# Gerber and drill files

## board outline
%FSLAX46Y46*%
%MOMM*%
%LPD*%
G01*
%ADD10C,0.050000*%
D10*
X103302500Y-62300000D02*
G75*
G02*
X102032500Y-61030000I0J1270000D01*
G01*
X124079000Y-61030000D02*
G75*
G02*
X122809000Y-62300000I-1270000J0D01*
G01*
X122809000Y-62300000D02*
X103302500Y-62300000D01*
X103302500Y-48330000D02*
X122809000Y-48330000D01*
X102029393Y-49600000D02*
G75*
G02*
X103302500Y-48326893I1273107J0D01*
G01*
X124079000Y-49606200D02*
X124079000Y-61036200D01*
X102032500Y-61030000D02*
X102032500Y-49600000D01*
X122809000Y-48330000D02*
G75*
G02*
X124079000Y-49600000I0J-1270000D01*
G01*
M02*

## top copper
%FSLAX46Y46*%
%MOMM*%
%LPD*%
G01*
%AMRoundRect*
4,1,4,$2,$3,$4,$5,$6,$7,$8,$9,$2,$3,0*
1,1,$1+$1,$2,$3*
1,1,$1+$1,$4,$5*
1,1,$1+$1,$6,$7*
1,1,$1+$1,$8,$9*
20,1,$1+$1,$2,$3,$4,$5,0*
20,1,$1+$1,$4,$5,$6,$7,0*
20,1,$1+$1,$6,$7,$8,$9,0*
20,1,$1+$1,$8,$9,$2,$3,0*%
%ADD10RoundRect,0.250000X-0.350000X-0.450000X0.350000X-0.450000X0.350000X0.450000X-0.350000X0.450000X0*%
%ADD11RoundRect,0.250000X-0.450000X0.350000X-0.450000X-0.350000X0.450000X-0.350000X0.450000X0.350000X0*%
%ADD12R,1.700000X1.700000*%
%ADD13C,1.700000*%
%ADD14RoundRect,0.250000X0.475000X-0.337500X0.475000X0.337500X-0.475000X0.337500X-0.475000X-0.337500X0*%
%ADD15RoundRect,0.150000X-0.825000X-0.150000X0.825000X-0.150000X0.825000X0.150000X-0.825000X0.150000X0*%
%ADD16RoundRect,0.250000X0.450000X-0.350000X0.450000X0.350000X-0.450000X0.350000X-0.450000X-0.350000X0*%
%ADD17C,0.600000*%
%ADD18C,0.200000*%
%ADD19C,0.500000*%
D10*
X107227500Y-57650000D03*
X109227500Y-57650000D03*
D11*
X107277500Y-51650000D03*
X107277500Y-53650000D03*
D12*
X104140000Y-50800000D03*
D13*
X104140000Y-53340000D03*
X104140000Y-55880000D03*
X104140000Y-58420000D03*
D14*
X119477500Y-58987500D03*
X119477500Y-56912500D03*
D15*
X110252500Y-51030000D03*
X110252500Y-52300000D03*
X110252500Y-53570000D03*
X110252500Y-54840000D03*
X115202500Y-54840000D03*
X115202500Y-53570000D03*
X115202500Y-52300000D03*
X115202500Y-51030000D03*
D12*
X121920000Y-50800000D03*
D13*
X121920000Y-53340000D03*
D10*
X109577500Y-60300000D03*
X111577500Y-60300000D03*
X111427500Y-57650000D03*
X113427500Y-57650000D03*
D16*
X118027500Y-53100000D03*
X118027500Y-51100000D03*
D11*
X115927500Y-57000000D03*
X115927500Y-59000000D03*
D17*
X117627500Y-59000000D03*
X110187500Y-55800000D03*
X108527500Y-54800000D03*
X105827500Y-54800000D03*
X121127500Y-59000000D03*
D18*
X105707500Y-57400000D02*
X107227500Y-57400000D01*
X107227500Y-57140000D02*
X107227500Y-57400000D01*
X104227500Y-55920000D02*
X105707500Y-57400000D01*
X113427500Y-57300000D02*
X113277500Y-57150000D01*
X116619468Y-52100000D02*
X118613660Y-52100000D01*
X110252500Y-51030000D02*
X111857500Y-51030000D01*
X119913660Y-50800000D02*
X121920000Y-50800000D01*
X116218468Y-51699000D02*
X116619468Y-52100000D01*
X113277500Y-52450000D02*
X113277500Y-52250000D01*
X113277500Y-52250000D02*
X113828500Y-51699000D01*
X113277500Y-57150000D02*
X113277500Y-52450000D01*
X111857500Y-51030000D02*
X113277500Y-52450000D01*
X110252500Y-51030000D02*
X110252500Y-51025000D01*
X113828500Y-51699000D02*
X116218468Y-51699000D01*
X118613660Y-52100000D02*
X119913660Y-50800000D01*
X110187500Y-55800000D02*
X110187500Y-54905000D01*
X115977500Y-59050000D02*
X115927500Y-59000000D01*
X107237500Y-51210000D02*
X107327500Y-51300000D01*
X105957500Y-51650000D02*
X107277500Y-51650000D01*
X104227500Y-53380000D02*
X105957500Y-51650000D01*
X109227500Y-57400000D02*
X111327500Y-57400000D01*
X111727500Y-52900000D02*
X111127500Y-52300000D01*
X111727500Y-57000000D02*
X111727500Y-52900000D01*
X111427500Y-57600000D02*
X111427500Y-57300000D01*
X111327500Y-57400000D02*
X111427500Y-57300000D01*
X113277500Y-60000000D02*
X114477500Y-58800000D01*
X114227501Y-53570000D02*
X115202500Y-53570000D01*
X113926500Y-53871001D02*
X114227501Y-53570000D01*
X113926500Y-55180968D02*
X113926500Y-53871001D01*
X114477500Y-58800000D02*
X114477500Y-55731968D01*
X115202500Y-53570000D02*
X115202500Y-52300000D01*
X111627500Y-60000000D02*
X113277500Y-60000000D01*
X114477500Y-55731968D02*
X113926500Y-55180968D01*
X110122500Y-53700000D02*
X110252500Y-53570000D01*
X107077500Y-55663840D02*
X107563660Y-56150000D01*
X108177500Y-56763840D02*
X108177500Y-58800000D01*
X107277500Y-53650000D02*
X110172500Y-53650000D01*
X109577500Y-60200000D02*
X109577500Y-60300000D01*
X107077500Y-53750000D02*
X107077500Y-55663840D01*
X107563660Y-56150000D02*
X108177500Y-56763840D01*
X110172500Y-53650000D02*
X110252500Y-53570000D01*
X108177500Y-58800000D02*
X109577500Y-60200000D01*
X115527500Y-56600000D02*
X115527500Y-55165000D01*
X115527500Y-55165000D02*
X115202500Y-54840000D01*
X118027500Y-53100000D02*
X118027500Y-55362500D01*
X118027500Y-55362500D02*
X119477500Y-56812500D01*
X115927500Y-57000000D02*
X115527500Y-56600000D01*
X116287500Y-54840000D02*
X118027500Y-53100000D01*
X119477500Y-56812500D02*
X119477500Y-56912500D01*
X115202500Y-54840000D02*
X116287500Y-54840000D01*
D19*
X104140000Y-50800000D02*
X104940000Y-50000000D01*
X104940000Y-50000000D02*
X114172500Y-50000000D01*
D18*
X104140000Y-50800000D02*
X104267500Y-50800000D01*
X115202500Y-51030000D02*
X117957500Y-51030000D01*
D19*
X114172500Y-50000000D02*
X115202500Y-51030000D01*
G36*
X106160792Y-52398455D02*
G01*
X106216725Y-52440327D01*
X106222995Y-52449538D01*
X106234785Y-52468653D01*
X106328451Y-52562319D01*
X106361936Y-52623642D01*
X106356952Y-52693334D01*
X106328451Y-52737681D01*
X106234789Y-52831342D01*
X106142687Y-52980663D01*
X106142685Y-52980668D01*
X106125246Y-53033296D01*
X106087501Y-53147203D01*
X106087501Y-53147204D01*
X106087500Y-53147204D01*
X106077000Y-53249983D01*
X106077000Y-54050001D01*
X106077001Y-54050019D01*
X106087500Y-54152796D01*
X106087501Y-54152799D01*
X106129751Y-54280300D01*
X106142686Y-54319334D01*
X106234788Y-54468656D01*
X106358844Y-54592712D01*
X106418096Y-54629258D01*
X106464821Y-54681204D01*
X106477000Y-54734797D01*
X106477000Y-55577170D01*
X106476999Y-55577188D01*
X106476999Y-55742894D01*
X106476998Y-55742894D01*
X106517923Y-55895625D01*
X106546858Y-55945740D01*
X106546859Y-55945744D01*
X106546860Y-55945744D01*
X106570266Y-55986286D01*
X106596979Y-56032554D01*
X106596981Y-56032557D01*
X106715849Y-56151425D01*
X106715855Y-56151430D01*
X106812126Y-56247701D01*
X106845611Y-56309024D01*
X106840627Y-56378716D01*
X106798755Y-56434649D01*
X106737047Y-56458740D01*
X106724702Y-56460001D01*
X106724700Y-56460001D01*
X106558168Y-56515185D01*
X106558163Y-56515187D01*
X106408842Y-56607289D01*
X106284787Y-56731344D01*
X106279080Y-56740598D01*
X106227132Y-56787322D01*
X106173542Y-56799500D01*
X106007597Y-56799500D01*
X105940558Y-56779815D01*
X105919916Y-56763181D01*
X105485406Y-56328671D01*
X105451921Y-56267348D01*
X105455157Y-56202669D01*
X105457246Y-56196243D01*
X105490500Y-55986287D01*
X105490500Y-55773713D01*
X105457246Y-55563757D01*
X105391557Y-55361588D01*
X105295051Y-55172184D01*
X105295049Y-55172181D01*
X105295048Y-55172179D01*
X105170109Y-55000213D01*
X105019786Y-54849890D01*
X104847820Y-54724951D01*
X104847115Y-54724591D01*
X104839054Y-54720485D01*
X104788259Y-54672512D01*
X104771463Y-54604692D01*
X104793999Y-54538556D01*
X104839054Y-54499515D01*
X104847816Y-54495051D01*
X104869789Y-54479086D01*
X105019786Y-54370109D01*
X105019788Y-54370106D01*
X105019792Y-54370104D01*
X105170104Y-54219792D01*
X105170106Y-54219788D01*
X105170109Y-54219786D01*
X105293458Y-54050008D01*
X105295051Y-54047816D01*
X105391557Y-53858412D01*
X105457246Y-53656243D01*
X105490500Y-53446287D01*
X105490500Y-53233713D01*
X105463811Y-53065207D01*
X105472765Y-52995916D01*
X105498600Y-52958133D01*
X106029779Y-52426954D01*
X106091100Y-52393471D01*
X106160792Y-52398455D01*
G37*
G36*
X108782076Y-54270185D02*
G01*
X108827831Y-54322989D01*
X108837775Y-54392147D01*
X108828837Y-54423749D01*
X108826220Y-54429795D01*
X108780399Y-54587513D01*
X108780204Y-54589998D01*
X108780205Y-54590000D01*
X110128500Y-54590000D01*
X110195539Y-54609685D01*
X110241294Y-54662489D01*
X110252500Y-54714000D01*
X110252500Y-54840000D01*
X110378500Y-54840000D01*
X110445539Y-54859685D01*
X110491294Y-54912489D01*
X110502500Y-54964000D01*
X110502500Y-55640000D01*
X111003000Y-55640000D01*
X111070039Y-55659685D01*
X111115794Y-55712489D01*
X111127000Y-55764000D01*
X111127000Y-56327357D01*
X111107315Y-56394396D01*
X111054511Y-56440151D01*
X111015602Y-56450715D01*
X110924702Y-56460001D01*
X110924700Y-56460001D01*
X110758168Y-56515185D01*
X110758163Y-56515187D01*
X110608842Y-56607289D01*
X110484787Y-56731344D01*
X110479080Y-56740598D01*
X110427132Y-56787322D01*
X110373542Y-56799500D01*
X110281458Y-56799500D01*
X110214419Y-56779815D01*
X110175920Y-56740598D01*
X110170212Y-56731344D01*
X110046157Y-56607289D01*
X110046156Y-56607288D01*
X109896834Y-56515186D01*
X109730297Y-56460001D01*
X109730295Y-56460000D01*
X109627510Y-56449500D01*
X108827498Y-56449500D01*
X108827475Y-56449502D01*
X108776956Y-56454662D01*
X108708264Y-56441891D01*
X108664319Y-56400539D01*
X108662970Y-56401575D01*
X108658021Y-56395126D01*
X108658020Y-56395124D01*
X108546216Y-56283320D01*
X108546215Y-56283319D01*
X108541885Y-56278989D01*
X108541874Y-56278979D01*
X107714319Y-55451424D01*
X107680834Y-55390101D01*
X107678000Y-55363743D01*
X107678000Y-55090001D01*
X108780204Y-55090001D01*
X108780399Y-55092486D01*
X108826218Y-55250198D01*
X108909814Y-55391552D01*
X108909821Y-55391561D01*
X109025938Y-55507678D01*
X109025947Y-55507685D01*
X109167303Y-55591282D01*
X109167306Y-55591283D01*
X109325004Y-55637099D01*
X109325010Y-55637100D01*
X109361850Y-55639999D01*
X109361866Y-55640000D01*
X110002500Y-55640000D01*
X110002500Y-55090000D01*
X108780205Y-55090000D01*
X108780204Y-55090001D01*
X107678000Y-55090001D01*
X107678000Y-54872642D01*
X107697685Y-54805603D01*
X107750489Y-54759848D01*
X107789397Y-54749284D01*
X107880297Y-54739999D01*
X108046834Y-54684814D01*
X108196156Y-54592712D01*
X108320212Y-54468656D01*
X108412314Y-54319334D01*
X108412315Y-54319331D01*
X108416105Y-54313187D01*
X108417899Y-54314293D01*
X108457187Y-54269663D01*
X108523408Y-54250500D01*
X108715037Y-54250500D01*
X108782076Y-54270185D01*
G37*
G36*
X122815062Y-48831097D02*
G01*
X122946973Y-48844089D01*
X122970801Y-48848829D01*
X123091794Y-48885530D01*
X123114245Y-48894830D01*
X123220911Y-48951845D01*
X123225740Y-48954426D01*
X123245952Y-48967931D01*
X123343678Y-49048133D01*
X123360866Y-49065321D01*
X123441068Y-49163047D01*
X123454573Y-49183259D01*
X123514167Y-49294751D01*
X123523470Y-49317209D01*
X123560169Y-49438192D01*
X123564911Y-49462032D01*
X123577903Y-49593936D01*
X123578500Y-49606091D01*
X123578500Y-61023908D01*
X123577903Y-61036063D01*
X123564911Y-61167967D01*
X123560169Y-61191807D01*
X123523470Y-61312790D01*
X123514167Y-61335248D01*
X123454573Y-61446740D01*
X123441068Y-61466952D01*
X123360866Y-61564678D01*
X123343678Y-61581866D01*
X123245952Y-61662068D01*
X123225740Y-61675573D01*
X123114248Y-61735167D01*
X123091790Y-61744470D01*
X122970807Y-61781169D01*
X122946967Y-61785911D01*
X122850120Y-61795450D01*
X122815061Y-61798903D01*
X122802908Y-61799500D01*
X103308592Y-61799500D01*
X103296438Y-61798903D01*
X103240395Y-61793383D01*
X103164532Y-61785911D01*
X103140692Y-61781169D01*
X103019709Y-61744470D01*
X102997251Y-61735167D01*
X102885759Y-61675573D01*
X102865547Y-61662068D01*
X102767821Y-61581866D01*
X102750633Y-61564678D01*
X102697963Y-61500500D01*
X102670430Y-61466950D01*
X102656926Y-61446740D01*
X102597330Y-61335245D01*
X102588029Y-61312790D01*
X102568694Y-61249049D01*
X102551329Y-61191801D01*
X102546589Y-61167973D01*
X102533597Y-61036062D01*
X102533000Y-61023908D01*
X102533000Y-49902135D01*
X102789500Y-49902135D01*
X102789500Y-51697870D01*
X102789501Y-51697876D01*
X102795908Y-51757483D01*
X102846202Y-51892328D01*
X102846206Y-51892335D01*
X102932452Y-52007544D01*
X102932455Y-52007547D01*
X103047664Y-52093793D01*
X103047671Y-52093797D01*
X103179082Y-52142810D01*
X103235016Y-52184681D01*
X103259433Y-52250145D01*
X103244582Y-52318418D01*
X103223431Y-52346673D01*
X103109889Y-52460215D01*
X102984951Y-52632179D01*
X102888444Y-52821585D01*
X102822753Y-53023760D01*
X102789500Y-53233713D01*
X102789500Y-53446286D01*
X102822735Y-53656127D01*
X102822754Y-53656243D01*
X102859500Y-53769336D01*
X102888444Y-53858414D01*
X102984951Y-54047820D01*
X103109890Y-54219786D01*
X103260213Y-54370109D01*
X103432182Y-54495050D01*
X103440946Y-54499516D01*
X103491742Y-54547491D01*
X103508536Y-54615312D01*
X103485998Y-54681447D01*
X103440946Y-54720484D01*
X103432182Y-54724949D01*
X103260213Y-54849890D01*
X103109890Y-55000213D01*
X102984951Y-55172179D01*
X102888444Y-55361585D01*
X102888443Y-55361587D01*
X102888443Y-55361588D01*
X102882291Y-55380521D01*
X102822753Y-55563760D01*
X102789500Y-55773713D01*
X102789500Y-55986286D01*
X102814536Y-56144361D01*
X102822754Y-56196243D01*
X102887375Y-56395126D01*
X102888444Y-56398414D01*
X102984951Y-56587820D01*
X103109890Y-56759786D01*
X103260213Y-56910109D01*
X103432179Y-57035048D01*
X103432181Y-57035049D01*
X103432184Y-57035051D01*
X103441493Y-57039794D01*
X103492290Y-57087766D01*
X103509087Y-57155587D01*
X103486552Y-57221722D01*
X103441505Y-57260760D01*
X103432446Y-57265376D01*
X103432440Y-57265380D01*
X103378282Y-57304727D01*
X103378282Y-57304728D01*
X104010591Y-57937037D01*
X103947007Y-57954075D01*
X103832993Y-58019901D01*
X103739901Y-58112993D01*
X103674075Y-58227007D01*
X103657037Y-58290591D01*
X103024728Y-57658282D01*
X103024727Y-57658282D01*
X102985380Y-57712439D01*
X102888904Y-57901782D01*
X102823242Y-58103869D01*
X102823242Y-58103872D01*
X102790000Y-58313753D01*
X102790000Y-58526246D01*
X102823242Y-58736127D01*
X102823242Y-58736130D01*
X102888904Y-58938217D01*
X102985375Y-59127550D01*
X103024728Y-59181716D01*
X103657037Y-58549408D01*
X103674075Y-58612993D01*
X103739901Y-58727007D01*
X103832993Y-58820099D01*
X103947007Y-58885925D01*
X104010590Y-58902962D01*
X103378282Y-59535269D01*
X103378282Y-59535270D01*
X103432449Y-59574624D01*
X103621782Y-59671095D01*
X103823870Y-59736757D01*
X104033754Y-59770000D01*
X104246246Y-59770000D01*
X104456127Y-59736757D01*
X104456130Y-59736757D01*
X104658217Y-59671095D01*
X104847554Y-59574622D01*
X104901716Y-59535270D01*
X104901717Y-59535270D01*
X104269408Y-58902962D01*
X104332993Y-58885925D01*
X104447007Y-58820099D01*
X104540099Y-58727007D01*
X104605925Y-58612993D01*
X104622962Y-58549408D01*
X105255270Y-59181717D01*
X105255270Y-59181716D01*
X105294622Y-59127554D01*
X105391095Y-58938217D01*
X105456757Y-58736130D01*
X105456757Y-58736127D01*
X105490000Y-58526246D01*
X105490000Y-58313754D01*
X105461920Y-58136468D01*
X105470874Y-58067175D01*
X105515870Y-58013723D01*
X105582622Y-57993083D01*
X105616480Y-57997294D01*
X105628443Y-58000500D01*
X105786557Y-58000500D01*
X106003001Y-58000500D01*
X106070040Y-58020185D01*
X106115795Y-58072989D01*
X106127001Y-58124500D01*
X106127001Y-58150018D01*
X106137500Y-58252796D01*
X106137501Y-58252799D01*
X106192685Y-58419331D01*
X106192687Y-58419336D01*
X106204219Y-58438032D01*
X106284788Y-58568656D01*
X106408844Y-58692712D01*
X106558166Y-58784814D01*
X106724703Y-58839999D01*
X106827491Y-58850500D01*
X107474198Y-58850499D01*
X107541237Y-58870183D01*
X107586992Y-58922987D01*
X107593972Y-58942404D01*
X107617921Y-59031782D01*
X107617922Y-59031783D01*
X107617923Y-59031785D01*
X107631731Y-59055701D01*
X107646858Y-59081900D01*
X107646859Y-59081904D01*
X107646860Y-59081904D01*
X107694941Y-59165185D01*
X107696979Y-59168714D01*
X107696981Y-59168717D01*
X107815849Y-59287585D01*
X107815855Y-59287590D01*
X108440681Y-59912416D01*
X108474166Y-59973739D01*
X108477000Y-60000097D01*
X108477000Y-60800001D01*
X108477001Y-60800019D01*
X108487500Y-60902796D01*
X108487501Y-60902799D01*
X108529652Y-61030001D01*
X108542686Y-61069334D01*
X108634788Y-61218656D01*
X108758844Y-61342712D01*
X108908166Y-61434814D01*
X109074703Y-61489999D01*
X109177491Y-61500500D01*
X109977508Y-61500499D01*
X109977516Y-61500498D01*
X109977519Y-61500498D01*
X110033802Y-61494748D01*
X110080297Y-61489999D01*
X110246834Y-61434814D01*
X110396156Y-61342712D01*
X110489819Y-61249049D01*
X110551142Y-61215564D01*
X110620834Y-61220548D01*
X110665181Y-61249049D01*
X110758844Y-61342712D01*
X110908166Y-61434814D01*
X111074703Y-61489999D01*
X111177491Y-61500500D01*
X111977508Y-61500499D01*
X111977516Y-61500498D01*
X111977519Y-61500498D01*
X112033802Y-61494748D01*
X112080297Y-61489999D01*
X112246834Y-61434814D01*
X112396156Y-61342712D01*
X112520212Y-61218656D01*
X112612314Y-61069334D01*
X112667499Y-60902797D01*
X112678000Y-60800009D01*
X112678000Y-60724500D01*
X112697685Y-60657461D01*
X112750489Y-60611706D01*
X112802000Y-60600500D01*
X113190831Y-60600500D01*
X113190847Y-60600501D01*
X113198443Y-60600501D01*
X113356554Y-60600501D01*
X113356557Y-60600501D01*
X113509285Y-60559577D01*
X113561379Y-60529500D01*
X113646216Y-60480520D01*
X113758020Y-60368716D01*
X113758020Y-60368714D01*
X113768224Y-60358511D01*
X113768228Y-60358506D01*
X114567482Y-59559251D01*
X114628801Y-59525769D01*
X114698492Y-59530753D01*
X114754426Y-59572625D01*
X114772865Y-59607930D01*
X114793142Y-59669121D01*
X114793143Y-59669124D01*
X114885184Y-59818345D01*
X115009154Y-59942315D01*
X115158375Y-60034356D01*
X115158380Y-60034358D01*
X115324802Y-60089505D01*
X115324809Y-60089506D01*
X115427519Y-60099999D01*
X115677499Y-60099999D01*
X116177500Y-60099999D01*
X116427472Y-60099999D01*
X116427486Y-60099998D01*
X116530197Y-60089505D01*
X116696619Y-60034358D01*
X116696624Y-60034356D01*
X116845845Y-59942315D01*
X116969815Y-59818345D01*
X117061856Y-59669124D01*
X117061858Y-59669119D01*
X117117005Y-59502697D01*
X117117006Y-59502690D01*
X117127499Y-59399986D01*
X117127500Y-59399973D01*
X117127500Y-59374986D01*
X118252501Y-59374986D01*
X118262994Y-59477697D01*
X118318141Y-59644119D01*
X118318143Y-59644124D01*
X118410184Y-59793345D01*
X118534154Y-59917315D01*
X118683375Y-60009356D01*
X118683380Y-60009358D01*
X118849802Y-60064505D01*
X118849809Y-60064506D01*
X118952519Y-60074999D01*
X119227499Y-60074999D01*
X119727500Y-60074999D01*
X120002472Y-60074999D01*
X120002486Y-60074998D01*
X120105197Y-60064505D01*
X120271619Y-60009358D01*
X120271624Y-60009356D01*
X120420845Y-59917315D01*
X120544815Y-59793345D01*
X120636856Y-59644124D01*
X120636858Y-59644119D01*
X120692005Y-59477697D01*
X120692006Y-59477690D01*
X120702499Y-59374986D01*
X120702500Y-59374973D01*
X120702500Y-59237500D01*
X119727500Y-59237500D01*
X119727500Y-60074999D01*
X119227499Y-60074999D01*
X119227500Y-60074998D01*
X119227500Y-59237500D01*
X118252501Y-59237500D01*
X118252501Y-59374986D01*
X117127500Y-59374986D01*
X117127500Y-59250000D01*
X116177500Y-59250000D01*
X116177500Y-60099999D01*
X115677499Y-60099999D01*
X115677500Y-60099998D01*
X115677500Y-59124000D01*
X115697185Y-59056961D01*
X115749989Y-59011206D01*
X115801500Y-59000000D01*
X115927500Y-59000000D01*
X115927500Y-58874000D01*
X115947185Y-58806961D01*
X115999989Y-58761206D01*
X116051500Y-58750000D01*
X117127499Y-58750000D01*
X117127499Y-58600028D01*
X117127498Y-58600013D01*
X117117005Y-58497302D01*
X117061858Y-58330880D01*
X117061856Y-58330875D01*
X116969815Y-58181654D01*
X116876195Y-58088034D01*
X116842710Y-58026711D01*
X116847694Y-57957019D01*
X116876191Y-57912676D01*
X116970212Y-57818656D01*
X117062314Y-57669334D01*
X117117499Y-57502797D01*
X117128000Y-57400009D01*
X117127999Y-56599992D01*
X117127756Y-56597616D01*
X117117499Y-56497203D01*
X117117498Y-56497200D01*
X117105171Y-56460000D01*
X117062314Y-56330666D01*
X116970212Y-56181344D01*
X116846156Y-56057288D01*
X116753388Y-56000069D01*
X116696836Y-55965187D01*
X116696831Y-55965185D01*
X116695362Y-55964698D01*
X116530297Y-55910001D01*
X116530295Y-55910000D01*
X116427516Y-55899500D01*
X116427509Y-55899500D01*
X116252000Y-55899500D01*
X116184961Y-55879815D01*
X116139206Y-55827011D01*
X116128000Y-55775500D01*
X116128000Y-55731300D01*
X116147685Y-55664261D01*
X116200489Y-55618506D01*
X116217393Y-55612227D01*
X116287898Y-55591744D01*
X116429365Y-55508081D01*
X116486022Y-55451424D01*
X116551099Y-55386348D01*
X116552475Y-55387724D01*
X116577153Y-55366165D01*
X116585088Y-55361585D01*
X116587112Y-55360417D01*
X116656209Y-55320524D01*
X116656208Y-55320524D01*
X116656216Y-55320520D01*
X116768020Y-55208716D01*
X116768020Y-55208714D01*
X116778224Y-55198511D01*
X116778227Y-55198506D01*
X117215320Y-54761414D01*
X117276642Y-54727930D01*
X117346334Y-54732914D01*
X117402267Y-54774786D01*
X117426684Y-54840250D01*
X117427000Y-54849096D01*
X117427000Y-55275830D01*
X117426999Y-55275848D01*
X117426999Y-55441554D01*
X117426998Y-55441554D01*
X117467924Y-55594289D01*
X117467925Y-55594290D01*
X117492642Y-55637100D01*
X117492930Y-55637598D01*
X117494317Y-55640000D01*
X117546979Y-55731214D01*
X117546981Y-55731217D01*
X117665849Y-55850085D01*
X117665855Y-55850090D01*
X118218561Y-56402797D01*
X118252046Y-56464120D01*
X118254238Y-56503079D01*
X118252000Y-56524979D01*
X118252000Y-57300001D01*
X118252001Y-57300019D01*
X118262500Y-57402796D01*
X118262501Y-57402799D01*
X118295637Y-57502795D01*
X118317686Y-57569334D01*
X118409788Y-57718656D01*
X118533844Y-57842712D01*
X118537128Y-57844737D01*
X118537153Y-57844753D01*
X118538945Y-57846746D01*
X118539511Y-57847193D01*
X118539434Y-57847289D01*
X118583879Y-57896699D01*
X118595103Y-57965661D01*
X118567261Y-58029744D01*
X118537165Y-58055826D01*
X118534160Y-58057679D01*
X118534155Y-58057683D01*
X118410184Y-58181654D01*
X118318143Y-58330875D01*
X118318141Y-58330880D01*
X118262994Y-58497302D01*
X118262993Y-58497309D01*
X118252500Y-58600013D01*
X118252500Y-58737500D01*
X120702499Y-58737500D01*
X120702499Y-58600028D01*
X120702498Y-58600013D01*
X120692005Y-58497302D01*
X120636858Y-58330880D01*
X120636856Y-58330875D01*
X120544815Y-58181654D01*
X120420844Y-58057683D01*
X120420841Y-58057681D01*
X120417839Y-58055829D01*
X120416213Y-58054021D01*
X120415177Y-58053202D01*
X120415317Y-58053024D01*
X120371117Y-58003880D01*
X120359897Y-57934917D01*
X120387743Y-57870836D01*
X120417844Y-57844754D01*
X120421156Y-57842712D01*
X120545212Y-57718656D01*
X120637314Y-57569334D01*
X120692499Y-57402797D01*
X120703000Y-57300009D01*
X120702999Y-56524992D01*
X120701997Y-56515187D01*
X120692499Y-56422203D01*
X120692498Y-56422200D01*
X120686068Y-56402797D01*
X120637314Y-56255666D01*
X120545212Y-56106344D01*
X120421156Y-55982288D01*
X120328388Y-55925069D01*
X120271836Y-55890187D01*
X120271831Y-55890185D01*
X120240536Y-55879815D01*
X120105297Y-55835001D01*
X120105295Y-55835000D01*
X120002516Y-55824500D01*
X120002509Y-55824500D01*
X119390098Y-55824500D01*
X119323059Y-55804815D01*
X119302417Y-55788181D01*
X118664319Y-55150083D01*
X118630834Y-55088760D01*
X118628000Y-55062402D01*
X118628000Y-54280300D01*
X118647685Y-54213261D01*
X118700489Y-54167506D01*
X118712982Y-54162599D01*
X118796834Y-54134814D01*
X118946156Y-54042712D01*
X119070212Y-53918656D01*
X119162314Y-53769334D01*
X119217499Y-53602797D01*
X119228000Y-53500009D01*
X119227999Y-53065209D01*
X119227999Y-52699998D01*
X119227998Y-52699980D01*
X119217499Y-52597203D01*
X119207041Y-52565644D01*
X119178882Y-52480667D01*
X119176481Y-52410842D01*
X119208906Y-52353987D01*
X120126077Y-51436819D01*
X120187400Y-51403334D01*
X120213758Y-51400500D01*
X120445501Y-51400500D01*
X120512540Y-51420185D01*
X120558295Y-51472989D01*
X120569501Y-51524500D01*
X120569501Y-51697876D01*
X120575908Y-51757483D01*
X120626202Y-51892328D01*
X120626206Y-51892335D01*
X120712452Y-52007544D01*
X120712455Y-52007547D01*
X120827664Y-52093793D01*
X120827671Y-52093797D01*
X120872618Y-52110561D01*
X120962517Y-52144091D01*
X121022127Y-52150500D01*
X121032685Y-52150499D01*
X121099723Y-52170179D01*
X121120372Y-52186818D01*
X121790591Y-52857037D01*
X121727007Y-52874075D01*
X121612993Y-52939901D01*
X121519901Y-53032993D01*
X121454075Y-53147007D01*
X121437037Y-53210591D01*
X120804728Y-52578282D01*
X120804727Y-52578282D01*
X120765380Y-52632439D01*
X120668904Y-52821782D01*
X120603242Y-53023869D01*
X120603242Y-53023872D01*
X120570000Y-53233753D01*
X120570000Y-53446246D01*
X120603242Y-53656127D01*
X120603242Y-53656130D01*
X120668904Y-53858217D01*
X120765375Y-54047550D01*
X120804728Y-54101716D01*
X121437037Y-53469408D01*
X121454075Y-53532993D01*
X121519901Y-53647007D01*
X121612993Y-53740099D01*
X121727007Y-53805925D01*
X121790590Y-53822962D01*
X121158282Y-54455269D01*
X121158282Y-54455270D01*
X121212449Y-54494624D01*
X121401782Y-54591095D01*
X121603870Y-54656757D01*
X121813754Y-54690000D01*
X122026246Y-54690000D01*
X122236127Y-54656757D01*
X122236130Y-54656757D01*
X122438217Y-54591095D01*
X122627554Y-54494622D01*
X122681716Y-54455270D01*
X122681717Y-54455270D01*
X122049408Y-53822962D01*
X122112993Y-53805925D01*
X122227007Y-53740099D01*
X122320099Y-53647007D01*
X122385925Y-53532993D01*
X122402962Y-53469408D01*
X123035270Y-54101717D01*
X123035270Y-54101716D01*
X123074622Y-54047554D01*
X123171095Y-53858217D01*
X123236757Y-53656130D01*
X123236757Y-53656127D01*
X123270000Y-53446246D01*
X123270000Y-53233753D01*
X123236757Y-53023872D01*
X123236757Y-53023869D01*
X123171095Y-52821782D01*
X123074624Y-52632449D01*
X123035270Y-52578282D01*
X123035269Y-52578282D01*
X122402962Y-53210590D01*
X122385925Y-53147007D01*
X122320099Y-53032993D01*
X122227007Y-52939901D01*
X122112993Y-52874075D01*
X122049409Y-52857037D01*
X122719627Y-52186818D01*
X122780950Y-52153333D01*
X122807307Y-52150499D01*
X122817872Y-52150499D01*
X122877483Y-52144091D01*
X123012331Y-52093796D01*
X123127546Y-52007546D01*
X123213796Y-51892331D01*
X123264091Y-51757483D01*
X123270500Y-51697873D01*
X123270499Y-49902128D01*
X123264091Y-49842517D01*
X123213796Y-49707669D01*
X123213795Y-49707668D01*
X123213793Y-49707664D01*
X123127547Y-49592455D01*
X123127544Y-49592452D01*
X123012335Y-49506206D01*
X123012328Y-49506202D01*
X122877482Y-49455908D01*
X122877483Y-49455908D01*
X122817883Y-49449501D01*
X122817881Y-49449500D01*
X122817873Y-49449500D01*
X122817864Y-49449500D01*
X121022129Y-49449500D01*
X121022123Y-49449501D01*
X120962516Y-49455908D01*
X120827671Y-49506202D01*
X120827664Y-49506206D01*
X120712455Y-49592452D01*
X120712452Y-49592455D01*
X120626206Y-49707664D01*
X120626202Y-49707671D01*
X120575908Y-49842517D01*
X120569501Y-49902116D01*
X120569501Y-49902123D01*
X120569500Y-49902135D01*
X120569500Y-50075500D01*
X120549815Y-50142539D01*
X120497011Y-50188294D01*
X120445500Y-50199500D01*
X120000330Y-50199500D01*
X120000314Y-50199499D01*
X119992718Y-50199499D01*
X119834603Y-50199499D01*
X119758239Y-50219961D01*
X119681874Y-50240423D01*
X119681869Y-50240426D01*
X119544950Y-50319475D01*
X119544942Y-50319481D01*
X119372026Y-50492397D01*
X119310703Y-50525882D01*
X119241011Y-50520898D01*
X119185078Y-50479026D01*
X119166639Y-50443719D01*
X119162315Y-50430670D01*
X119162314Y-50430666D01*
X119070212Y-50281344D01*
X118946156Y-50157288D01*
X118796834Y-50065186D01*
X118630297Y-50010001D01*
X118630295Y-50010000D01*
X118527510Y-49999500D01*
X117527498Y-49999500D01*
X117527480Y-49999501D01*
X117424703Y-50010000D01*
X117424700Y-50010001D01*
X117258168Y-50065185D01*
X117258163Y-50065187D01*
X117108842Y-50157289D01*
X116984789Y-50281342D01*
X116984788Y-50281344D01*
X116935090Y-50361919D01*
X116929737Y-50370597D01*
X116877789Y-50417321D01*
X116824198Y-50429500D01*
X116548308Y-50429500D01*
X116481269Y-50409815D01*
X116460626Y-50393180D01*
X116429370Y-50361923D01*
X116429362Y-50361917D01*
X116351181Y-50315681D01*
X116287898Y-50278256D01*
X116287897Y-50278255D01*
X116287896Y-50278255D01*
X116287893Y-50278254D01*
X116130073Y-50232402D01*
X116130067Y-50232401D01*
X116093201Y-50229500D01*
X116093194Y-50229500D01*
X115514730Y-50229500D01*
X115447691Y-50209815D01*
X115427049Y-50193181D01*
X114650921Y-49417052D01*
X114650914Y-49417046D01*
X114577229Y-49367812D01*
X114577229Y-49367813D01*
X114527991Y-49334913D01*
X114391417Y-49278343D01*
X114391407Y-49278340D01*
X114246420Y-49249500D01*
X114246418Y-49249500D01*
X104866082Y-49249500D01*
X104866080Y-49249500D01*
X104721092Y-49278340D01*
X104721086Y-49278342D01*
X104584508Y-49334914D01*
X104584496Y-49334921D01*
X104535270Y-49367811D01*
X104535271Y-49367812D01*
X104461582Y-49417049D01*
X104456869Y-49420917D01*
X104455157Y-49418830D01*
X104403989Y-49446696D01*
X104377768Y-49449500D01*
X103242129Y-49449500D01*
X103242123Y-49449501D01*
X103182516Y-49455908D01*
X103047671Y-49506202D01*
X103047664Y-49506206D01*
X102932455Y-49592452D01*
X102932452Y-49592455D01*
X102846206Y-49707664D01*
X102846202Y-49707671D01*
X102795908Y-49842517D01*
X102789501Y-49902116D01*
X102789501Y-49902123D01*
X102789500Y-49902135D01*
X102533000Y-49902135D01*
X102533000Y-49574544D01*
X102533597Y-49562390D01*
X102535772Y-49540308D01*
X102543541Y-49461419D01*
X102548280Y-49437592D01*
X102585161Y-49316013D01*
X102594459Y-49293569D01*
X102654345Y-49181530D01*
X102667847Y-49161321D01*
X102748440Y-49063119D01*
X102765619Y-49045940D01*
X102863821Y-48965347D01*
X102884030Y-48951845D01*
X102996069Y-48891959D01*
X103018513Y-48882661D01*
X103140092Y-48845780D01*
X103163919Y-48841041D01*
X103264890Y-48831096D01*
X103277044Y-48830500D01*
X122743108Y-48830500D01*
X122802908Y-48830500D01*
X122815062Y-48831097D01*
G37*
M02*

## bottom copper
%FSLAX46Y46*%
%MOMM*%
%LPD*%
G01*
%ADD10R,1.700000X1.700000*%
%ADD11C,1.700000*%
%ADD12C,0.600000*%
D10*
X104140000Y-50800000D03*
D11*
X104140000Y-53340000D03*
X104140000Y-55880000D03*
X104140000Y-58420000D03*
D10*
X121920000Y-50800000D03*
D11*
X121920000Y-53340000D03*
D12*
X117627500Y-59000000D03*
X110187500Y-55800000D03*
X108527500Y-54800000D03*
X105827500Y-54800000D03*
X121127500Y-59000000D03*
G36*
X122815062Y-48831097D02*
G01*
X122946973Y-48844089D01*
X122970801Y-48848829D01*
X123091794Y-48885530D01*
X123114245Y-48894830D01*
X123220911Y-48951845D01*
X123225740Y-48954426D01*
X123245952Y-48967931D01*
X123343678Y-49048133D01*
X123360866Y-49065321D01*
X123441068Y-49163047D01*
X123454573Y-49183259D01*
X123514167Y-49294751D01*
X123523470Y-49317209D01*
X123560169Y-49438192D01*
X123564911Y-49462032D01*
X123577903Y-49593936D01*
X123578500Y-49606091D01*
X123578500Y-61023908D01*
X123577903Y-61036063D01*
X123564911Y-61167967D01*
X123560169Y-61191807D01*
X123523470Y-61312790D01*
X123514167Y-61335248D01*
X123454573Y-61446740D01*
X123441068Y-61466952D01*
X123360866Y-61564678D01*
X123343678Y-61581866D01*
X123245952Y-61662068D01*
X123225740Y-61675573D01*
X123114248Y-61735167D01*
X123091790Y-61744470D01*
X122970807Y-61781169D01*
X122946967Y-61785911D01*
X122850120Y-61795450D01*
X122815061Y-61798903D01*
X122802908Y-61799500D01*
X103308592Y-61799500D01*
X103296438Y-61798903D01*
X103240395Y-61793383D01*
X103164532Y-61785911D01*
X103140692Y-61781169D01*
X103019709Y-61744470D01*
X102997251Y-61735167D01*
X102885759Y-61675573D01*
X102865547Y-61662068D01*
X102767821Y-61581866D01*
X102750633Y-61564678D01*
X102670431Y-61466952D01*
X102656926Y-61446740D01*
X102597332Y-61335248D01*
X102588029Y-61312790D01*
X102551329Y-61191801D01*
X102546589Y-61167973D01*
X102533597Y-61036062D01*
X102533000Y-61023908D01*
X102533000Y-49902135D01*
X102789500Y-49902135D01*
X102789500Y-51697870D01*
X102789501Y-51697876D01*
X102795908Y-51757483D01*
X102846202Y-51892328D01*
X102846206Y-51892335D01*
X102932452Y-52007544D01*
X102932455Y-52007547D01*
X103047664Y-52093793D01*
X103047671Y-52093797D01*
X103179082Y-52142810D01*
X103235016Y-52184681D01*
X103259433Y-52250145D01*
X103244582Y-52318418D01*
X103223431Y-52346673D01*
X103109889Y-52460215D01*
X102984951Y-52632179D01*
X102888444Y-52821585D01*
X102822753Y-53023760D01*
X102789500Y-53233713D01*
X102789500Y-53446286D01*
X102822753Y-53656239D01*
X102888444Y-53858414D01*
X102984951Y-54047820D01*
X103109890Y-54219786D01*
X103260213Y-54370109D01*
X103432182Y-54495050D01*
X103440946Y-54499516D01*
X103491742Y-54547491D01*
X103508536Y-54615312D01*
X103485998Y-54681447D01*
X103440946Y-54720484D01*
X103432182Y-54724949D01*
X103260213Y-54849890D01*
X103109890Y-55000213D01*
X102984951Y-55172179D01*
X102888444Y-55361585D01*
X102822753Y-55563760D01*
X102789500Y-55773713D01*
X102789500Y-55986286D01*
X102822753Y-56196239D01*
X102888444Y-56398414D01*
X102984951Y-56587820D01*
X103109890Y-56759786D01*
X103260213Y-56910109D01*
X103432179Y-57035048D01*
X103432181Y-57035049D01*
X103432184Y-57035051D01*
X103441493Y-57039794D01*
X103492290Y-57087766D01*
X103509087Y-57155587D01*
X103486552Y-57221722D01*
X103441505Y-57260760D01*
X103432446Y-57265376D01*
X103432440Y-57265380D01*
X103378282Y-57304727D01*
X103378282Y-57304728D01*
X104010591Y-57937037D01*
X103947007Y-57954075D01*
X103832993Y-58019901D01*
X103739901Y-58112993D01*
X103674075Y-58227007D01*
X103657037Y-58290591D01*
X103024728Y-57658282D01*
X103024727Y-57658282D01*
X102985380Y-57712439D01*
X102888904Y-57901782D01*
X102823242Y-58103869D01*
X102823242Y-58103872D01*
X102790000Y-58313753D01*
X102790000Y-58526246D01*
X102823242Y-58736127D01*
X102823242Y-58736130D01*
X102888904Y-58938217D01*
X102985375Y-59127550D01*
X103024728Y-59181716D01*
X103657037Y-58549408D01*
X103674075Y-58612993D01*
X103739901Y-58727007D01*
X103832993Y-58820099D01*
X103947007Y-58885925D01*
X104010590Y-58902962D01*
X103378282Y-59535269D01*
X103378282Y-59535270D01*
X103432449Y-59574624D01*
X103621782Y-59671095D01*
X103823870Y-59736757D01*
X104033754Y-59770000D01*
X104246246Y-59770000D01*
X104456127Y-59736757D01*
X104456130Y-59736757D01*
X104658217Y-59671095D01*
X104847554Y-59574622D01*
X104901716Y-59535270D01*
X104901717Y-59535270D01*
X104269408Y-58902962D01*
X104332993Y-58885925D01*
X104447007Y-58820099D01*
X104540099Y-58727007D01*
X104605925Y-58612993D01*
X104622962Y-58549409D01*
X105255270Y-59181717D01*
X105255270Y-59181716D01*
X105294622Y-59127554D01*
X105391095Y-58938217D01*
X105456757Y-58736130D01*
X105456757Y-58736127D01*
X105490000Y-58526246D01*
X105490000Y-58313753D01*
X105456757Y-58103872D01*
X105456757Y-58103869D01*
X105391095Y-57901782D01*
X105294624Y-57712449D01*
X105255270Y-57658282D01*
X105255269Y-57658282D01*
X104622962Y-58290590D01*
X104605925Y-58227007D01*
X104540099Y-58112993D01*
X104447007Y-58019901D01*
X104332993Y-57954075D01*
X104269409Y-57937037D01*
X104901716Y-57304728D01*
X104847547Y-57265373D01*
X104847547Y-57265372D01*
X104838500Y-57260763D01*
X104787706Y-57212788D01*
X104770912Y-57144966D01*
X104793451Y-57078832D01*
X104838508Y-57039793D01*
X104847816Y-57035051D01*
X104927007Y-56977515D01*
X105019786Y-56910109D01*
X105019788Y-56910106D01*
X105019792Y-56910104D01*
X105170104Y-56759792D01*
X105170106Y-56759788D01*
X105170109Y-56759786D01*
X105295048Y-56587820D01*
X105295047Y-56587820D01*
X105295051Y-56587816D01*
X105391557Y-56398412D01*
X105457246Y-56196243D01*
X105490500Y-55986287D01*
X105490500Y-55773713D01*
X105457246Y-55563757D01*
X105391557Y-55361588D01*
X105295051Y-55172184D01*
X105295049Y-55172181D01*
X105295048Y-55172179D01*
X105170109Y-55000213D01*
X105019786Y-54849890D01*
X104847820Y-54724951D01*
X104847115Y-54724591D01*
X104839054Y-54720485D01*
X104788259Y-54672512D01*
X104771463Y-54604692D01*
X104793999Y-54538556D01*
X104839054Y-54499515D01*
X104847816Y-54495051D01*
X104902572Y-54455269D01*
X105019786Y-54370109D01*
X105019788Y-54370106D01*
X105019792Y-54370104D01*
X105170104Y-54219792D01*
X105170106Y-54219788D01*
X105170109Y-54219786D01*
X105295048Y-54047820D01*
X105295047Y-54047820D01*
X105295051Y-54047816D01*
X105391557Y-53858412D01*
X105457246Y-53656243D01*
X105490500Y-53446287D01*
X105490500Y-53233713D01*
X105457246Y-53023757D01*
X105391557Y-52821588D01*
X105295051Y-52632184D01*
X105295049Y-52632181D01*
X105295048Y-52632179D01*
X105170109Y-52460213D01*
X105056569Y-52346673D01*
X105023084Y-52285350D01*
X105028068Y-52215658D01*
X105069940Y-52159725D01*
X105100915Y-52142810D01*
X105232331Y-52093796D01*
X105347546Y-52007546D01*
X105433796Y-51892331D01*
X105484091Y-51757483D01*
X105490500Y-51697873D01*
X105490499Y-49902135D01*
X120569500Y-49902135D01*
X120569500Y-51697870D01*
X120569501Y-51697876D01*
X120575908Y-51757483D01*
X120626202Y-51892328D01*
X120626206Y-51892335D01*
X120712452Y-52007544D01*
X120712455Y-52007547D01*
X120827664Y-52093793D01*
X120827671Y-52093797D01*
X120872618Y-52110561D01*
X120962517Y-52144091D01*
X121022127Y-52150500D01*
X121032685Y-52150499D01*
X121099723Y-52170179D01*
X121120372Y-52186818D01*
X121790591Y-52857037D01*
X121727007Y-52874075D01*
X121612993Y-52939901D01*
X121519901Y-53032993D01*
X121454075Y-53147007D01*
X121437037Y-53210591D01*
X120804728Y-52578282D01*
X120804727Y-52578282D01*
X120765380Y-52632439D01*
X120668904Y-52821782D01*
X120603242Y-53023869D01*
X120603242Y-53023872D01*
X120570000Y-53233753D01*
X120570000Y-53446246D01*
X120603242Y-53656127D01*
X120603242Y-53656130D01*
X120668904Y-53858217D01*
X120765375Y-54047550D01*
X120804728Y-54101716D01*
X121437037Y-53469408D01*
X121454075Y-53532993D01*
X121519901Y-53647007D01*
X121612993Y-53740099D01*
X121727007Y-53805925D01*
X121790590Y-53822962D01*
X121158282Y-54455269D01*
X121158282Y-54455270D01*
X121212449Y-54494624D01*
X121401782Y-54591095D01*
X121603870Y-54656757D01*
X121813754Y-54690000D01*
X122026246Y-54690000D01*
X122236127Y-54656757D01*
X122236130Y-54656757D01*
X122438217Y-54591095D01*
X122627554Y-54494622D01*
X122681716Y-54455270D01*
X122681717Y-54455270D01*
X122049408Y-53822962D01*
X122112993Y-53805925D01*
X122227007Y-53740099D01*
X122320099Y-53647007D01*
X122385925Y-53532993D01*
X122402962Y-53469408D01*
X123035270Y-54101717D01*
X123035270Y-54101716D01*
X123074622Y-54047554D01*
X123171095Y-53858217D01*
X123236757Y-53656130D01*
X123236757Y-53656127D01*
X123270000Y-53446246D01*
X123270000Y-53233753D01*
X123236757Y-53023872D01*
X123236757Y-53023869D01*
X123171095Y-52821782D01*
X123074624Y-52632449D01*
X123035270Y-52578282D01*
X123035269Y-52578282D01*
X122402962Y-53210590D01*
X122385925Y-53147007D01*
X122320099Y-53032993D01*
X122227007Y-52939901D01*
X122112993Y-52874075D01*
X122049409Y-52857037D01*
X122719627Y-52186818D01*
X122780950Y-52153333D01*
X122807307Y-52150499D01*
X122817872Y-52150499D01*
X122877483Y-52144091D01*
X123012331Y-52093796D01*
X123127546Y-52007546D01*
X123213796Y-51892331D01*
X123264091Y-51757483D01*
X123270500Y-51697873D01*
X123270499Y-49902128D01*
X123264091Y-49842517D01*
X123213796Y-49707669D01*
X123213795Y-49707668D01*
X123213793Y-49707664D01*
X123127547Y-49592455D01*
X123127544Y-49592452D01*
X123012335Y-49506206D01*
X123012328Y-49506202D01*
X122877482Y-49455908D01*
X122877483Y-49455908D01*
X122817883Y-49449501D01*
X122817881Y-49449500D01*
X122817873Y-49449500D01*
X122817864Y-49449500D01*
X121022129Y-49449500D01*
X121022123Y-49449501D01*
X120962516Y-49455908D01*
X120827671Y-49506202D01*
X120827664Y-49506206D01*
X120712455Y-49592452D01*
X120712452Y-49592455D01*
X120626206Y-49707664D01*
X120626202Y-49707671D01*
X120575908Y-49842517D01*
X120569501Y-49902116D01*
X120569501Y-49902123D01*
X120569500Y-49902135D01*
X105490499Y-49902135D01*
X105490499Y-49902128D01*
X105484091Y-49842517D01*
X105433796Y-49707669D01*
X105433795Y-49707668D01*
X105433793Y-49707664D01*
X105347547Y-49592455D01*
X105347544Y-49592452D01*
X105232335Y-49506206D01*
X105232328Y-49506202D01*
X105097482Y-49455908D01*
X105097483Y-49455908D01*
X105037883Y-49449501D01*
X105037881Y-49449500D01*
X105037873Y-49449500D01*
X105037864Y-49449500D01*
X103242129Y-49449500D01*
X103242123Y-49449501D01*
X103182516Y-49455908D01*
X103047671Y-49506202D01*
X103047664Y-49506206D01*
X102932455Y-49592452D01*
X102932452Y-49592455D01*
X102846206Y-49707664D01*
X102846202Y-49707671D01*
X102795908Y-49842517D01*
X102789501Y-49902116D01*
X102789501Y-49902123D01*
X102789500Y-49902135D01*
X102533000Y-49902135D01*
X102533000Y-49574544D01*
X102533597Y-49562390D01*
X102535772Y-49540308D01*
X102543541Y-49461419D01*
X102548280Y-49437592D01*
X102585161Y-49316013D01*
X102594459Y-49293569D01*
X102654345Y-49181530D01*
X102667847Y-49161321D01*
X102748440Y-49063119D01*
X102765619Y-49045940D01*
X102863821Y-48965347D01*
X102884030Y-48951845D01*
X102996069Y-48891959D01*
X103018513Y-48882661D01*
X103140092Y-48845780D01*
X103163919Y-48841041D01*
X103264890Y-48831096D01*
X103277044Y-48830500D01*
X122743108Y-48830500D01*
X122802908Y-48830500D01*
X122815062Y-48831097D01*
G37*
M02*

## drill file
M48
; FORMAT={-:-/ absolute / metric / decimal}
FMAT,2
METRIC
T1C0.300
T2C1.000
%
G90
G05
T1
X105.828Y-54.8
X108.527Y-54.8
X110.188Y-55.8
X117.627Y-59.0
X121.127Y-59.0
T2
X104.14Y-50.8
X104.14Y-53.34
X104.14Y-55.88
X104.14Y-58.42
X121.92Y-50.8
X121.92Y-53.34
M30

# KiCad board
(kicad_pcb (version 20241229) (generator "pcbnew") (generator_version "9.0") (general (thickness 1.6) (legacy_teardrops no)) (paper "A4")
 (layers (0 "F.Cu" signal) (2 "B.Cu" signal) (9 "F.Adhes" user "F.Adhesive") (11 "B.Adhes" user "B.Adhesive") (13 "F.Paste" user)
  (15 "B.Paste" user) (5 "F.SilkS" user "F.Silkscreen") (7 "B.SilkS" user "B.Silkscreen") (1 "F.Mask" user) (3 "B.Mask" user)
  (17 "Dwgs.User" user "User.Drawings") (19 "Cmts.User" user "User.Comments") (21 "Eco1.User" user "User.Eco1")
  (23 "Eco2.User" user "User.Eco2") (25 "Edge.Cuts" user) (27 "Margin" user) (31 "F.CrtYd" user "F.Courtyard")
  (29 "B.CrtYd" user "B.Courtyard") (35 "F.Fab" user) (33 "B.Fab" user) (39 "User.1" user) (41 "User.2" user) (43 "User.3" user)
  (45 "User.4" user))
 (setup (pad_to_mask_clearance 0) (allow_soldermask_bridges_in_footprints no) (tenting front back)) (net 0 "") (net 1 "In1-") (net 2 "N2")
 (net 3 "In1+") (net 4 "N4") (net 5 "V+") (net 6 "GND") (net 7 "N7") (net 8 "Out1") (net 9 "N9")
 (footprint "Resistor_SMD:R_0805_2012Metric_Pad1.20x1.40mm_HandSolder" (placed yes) (layer "F.Cu") (at 108.2275 57.65)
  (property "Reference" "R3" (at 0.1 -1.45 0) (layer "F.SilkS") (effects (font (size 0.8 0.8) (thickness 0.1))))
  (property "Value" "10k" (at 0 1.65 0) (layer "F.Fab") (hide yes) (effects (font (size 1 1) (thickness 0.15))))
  (pad "1" smd roundrect (at -1 0) (size 1.2 1.4) (layers "F.Cu" "F.Mask" "F.Paste") (roundrect_rratio 0.208333) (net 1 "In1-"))
  (pad "2" smd roundrect (at 1 0) (size 1.2 1.4) (layers "F.Cu" "F.Mask" "F.Paste") (roundrect_rratio 0.208333) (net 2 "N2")))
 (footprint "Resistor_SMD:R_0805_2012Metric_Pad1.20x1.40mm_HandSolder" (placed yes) (layer "F.Cu") (at 107.2775 52.65 -90)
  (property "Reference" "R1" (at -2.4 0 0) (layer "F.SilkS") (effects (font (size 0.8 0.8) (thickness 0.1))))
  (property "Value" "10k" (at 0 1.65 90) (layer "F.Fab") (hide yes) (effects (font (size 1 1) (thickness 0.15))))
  (pad "1" smd roundrect (at -1 0 270) (size 1.2 1.4) (layers "F.Cu" "F.Mask" "F.Paste") (roundrect_rratio 0.208333) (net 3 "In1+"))
  (pad "2" smd roundrect (at 1 0 270) (size 1.2 1.4) (layers "F.Cu" "F.Mask" "F.Paste") (roundrect_rratio 0.208333) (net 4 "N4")))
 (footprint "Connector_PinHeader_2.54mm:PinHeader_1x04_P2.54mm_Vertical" (layer "F.Cu") (at 104.14 50.8)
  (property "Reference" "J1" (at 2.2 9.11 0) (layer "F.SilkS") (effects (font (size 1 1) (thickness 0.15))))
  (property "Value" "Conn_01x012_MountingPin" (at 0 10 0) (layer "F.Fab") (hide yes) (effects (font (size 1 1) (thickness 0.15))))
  (pad "1" thru_hole rect (at 0 0) (size 1.7 1.7) (drill 1) (layers "*.Cu" "*.Mask") (remove_unused_layers no) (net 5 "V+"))
  (pad "2" thru_hole circle (at 0 2.54) (size 1.7 1.7) (drill 1) (layers "*.Cu" "*.Mask") (remove_unused_layers no) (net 3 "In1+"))
  (pad "3" thru_hole circle (at 0 5.08) (size 1.7 1.7) (drill 1) (layers "*.Cu" "*.Mask") (remove_unused_layers no) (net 1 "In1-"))
  (pad "4" thru_hole circle (at 0 7.62) (size 1.7 1.7) (drill 1) (layers "*.Cu" "*.Mask") (remove_unused_layers no) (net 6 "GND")))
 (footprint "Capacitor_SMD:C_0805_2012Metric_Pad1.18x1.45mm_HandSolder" (layer "F.Cu") (at 119.4775 57.95 90)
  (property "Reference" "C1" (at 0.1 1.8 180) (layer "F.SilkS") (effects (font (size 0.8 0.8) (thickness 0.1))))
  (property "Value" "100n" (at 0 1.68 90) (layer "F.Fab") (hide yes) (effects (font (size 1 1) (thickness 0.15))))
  (pad "1" smd roundrect (at -1.0375 0 90) (size 1.175 1.45) (layers "F.Cu" "F.Mask" "F.Paste") (roundrect_rratio 0.212766) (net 6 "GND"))
  (pad "2" smd roundrect (at 1.0375 0 90) (size 1.175 1.45) (layers "F.Cu" "F.Mask" "F.Paste") (roundrect_rratio 0.212766) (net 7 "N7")))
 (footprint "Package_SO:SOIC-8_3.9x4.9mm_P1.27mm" (layer "F.Cu") (at 112.7275 52.935)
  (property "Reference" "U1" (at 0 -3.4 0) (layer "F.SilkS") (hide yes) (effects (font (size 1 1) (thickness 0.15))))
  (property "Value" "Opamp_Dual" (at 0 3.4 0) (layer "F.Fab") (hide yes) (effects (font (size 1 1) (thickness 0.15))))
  (pad "1" smd roundrect (at -2.475 -1.905) (size 1.95 0.6) (layers "F.Cu" "F.Mask" "F.Paste") (roundrect_rratio 0.25) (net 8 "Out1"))
  (pad "2" smd roundrect (at -2.475 -0.635) (size 1.95 0.6) (layers "F.Cu" "F.Mask" "F.Paste") (roundrect_rratio 0.25) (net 2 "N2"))
  (pad "3" smd roundrect (at -2.475 0.635) (size 1.95 0.6) (layers "F.Cu" "F.Mask" "F.Paste") (roundrect_rratio 0.25) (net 4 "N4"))
  (pad "4" smd roundrect (at -2.475 1.905) (size 1.95 0.6) (layers "F.Cu" "F.Mask" "F.Paste") (roundrect_rratio 0.25) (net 6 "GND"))
  (pad "5" smd roundrect (at 2.475 1.905) (size 1.95 0.6) (layers "F.Cu" "F.Mask" "F.Paste") (roundrect_rratio 0.25) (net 7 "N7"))
  (pad "6" smd roundrect (at 2.475 0.635) (size 1.95 0.6) (layers "F.Cu" "F.Mask" "F.Paste") (roundrect_rratio 0.25) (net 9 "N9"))
  (pad "7" smd roundrect (at 2.475 -0.635) (size 1.95 0.6) (layers "F.Cu" "F.Mask" "F.Paste") (roundrect_rratio 0.25) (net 9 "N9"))
  (pad "8" smd roundrect (at 2.475 -1.905) (size 1.95 0.6) (layers "F.Cu" "F.Mask" "F.Paste") (roundrect_rratio 0.25) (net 5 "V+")))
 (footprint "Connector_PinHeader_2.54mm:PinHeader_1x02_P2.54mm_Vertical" (layer "F.Cu") (at 121.92 50.8)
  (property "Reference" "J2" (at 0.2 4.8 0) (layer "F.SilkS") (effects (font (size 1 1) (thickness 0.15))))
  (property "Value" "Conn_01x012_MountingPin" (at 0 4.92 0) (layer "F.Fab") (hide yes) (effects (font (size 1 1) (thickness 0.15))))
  (pad "1" thru_hole rect (at 0 0) (size 1.7 1.7) (drill 1) (layers "*.Cu" "*.Mask") (remove_unused_layers no) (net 8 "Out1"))
  (pad "2" thru_hole circle (at 0 2.54) (size 1.7 1.7) (drill 1) (layers "*.Cu" "*.Mask") (remove_unused_layers no) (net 6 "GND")))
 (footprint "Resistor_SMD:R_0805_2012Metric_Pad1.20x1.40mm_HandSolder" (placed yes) (layer "F.Cu") (at 110.5775 60.3)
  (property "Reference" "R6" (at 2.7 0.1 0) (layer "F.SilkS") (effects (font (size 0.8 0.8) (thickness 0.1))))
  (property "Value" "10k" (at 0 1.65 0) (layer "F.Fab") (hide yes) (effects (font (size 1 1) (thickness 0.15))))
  (pad "1" smd roundrect (at -1 0) (size 1.2 1.4) (layers "F.Cu" "F.Mask" "F.Paste") (roundrect_rratio 0.208333) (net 4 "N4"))
  (pad "2" smd roundrect (at 1 0) (size 1.2 1.4) (layers "F.Cu" "F.Mask" "F.Paste") (roundrect_rratio 0.208333) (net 9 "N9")))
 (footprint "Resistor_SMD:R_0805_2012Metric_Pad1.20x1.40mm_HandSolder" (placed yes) (layer "F.Cu") (at 112.4275 57.65)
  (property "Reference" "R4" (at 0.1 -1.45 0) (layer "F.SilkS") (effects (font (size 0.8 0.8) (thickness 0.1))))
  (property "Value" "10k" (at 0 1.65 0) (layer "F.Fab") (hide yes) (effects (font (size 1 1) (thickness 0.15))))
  (pad "1" smd roundrect (at -1 0) (size 1.2 1.4) (layers "F.Cu" "F.Mask" "F.Paste") (roundrect_rratio 0.208333) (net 2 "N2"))
  (pad "2" smd roundrect (at 1 0) (size 1.2 1.4) (layers "F.Cu" "F.Mask" "F.Paste") (roundrect_rratio 0.208333) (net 8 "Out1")))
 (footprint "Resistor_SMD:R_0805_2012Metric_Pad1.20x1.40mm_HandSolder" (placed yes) (layer "F.Cu") (at 118.0275 52.1 90)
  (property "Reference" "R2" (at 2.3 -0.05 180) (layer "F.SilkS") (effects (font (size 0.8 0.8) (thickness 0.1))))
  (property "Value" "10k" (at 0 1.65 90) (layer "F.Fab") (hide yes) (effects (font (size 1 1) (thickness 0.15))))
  (pad "1" smd roundrect (at -1 0 90) (size 1.2 1.4) (layers "F.Cu" "F.Mask" "F.Paste") (roundrect_rratio 0.208333) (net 7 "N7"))
  (pad "2" smd roundrect (at 1 0 90) (size 1.2 1.4) (layers "F.Cu" "F.Mask" "F.Paste") (roundrect_rratio 0.208333) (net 5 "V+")))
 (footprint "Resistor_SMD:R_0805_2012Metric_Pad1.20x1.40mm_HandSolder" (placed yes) (layer "F.Cu") (at 115.9275 58 -90)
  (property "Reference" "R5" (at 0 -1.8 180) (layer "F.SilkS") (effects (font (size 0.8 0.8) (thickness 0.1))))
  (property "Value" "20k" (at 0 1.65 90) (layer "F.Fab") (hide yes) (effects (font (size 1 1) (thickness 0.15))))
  (pad "1" smd roundrect (at -1 0 270) (size 1.2 1.4) (layers "F.Cu" "F.Mask" "F.Paste") (roundrect_rratio 0.208333) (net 7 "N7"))
  (pad "2" smd roundrect (at 1 0 270) (size 1.2 1.4) (layers "F.Cu" "F.Mask" "F.Paste") (roundrect_rratio 0.208333) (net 6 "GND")))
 (gr_arc (start 103.3025 62.3) (mid 102.404474 61.928026) (end 102.0325 61.03) (stroke (width 0.05) (type default)) (layer "Edge.Cuts"))
 (gr_arc (start 124.079 61.03) (mid 123.707026 61.928026) (end 122.809 62.3) (stroke (width 0.05) (type default)) (layer "Edge.Cuts"))
 (gr_line (start 122.809 62.3) (end 103.3025 62.3) (stroke (width 0.05) (type default)) (layer "Edge.Cuts"))
 (gr_line (start 103.3025 48.33) (end 122.809 48.33) (stroke (width 0.05) (type default)) (layer "Edge.Cuts"))
 (gr_arc (start 102.029393 49.6) (mid 102.402277 48.699777) (end 103.3025 48.326893) (stroke (width 0.05) (type default))
  (layer "Edge.Cuts"))
 (gr_line (start 124.079 49.6062) (end 124.079 61.0362) (stroke (width 0.05) (type default)) (layer "Edge.Cuts"))
 (gr_line (start 102.0325 61.03) (end 102.0325 49.6) (stroke (width 0.05) (type default)) (layer "Edge.Cuts"))
 (gr_arc (start 122.809 48.33) (mid 123.707026 48.701974) (end 124.079 49.6) (stroke (width 0.05) (type default)) (layer "Edge.Cuts"))
 (segment (start 105.7075 57.4) (end 107.2275 57.4) (width 0.2) (layer "F.Cu") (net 1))
 (segment (start 107.2275 57.14) (end 107.2275 57.4) (width 0.2) (layer "F.Cu") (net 1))
 (segment (start 104.2275 55.92) (end 105.7075 57.4) (width 0.2) (layer "F.Cu") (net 1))
 (segment (start 113.4275 57.3) (end 113.2775 57.15) (width 0.2) (layer "F.Cu") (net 8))
 (segment (start 116.619468 52.1) (end 118.61366 52.1) (width 0.2) (layer "F.Cu") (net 8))
 (segment (start 110.2525 51.03) (end 111.8575 51.03) (width 0.2) (layer "F.Cu") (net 8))
 (segment (start 119.91366 50.8) (end 121.92 50.8) (width 0.2) (layer "F.Cu") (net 8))
 (segment (start 116.218468 51.699) (end 116.619468 52.1) (width 0.2) (layer "F.Cu") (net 8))
 (segment (start 113.2775 52.45) (end 113.2775 52.25) (width 0.2) (layer "F.Cu") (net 8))
 (segment (start 113.2775 52.25) (end 113.8285 51.699) (width 0.2) (layer "F.Cu") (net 8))
 (segment (start 113.2775 57.15) (end 113.2775 52.45) (width 0.2) (layer "F.Cu") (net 8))
 (segment (start 111.8575 51.03) (end 113.2775 52.45) (width 0.2) (layer "F.Cu") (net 8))
 (segment (start 110.2525 51.03) (end 110.2525 51.025) (width 0.2) (layer "F.Cu") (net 8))
 (segment (start 113.8285 51.699) (end 116.218468 51.699) (width 0.2) (layer "F.Cu") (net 8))
 (segment (start 118.61366 52.1) (end 119.91366 50.8) (width 0.2) (layer "F.Cu") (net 8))
 (segment (start 110.1875 55.8) (end 110.1875 54.905) (width 0.2) (layer "F.Cu") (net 6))
 (segment (start 115.9775 59.05) (end 115.9275 59) (width 0.2) (layer "F.Cu") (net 6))
 (via (at 117.6275 59) (size 0.6) (drill 0.3) (layers "F.Cu" "B.Cu") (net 6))
 (via (at 110.1875 55.8) (size 0.6) (drill 0.3) (layers "F.Cu" "B.Cu") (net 6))
 (via (at 108.5275 54.8) (size 0.6) (drill 0.3) (layers "F.Cu" "B.Cu") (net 6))
 (via (at 105.8275 54.8) (size 0.6) (drill 0.3) (layers "F.Cu" "B.Cu") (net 6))
 (via (at 121.1275 59) (size 0.6) (drill 0.3) (layers "F.Cu" "B.Cu") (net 6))
 (segment (start 107.2375 51.21) (end 107.3275 51.3) (width 0.2) (layer "F.Cu") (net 3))
 (segment (start 105.9575 51.65) (end 107.2775 51.65) (width 0.2) (layer "F.Cu") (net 3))
 (segment (start 104.2275 53.38) (end 105.9575 51.65) (width 0.2) (layer "F.Cu") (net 3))
 (segment (start 109.2275 57.4) (end 111.3275 57.4) (width 0.2) (layer "F.Cu") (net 2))
 (segment (start 111.7275 52.9) (end 111.1275 52.3) (width 0.2) (layer "F.Cu") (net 2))
 (segment (start 111.7275 57) (end 111.7275 52.9) (width 0.2) (layer "F.Cu") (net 2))
 (segment (start 111.4275 57.6) (end 111.4275 57.3) (width 0.2) (layer "F.Cu") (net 2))
 (segment (start 111.3275 57.4) (end 111.4275 57.3) (width 0.2) (layer "F.Cu") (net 2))
 (segment (start 113.2775 60) (end 114.4775 58.8) (width 0.2) (layer "F.Cu") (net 9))
 (segment (start 114.227501 53.57) (end 115.2025 53.57) (width 0.2) (layer "F.Cu") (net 9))
 (segment (start 113.9265 53.871001) (end 114.227501 53.57) (width 0.2) (layer "F.Cu") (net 9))
 (segment (start 113.9265 55.180968) (end 113.9265 53.871001) (width 0.2) (layer "F.Cu") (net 9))
 (segment (start 114.4775 58.8) (end 114.4775 55.731968) (width 0.2) (layer "F.Cu") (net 9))
 (segment (start 115.2025 53.57) (end 115.2025 52.3) (width 0.2) (layer "F.Cu") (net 9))
 (segment (start 111.6275 60) (end 113.2775 60) (width 0.2) (layer "F.Cu") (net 9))
 (segment (start 114.4775 55.731968) (end 113.9265 55.180968) (width 0.2) (layer "F.Cu") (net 9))
 (segment (start 110.1225 53.7) (end 110.2525 53.57) (width 0.2) (layer "F.Cu") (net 4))
 (segment (start 107.0775 55.66384) (end 107.56366 56.15) (width 0.2) (layer "F.Cu") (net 4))
 (segment (start 108.1775 56.76384) (end 108.1775 58.8) (width 0.2) (layer "F.Cu") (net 4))
 (segment (start 107.2775 53.65) (end 110.1725 53.65) (width 0.2) (layer "F.Cu") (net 4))
 (segment (start 109.5775 60.2) (end 109.5775 60.3) (width 0.2) (layer "F.Cu") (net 4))
 (segment (start 107.0775 53.75) (end 107.0775 55.66384) (width 0.2) (layer "F.Cu") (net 4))
 (segment (start 107.56366 56.15) (end 108.1775 56.76384) (width 0.2) (layer "F.Cu") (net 4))
 (segment (start 110.1725 53.65) (end 110.2525 53.57) (width 0.2) (layer "F.Cu") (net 4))
 (segment (start 108.1775 58.8) (end 109.5775 60.2) (width 0.2) (layer "F.Cu") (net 4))
 (segment (start 115.5275 56.6) (end 115.5275 55.165) (width 0.2) (layer "F.Cu") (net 7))
 (segment (start 115.5275 55.165) (end 115.2025 54.84) (width 0.2) (layer "F.Cu") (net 7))
 (segment (start 118.0275 53.1) (end 118.0275 55.3625) (width 0.2) (layer "F.Cu") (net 7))
 (segment (start 118.0275 55.3625) (end 119.4775 56.8125) (width 0.2) (layer "F.Cu") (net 7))
 (segment (start 115.9275 57) (end 115.5275 56.6) (width 0.2) (layer "F.Cu") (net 7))
 (segment (start 116.2875 54.84) (end 118.0275 53.1) (width 0.2) (layer "F.Cu") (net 7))
 (segment (start 119.4775 56.8125) (end 119.4775 56.9125) (width 0.2) (layer "F.Cu") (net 7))
 (segment (start 115.2025 54.84) (end 116.2875 54.84) (width 0.2) (layer "F.Cu") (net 7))
 (segment (start 104.14 50.8) (end 104.94 50) (width 0.5) (layer "F.Cu") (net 5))
 (segment (start 104.94 50) (end 114.1725 50) (width 0.5) (layer "F.Cu") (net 5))
 (segment (start 104.14 50.8) (end 104.2675 50.8) (width 0.2) (layer "F.Cu") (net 5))
 (segment (start 115.2025 51.03) (end 117.9575 51.03) (width 0.2) (layer "F.Cu") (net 5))
 (segment (start 114.1725 50) (end 115.2025 51.03) (width 0.5) (layer "F.Cu") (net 5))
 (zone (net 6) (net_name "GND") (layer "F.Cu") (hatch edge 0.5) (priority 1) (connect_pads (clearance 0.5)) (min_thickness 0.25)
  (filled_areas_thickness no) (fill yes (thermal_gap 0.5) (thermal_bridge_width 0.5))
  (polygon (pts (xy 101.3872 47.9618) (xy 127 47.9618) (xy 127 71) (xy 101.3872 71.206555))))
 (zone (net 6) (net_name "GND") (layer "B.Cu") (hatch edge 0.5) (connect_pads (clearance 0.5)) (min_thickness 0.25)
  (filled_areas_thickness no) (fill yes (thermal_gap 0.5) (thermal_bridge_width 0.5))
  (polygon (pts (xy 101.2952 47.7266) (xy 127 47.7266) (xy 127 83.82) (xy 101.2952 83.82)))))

